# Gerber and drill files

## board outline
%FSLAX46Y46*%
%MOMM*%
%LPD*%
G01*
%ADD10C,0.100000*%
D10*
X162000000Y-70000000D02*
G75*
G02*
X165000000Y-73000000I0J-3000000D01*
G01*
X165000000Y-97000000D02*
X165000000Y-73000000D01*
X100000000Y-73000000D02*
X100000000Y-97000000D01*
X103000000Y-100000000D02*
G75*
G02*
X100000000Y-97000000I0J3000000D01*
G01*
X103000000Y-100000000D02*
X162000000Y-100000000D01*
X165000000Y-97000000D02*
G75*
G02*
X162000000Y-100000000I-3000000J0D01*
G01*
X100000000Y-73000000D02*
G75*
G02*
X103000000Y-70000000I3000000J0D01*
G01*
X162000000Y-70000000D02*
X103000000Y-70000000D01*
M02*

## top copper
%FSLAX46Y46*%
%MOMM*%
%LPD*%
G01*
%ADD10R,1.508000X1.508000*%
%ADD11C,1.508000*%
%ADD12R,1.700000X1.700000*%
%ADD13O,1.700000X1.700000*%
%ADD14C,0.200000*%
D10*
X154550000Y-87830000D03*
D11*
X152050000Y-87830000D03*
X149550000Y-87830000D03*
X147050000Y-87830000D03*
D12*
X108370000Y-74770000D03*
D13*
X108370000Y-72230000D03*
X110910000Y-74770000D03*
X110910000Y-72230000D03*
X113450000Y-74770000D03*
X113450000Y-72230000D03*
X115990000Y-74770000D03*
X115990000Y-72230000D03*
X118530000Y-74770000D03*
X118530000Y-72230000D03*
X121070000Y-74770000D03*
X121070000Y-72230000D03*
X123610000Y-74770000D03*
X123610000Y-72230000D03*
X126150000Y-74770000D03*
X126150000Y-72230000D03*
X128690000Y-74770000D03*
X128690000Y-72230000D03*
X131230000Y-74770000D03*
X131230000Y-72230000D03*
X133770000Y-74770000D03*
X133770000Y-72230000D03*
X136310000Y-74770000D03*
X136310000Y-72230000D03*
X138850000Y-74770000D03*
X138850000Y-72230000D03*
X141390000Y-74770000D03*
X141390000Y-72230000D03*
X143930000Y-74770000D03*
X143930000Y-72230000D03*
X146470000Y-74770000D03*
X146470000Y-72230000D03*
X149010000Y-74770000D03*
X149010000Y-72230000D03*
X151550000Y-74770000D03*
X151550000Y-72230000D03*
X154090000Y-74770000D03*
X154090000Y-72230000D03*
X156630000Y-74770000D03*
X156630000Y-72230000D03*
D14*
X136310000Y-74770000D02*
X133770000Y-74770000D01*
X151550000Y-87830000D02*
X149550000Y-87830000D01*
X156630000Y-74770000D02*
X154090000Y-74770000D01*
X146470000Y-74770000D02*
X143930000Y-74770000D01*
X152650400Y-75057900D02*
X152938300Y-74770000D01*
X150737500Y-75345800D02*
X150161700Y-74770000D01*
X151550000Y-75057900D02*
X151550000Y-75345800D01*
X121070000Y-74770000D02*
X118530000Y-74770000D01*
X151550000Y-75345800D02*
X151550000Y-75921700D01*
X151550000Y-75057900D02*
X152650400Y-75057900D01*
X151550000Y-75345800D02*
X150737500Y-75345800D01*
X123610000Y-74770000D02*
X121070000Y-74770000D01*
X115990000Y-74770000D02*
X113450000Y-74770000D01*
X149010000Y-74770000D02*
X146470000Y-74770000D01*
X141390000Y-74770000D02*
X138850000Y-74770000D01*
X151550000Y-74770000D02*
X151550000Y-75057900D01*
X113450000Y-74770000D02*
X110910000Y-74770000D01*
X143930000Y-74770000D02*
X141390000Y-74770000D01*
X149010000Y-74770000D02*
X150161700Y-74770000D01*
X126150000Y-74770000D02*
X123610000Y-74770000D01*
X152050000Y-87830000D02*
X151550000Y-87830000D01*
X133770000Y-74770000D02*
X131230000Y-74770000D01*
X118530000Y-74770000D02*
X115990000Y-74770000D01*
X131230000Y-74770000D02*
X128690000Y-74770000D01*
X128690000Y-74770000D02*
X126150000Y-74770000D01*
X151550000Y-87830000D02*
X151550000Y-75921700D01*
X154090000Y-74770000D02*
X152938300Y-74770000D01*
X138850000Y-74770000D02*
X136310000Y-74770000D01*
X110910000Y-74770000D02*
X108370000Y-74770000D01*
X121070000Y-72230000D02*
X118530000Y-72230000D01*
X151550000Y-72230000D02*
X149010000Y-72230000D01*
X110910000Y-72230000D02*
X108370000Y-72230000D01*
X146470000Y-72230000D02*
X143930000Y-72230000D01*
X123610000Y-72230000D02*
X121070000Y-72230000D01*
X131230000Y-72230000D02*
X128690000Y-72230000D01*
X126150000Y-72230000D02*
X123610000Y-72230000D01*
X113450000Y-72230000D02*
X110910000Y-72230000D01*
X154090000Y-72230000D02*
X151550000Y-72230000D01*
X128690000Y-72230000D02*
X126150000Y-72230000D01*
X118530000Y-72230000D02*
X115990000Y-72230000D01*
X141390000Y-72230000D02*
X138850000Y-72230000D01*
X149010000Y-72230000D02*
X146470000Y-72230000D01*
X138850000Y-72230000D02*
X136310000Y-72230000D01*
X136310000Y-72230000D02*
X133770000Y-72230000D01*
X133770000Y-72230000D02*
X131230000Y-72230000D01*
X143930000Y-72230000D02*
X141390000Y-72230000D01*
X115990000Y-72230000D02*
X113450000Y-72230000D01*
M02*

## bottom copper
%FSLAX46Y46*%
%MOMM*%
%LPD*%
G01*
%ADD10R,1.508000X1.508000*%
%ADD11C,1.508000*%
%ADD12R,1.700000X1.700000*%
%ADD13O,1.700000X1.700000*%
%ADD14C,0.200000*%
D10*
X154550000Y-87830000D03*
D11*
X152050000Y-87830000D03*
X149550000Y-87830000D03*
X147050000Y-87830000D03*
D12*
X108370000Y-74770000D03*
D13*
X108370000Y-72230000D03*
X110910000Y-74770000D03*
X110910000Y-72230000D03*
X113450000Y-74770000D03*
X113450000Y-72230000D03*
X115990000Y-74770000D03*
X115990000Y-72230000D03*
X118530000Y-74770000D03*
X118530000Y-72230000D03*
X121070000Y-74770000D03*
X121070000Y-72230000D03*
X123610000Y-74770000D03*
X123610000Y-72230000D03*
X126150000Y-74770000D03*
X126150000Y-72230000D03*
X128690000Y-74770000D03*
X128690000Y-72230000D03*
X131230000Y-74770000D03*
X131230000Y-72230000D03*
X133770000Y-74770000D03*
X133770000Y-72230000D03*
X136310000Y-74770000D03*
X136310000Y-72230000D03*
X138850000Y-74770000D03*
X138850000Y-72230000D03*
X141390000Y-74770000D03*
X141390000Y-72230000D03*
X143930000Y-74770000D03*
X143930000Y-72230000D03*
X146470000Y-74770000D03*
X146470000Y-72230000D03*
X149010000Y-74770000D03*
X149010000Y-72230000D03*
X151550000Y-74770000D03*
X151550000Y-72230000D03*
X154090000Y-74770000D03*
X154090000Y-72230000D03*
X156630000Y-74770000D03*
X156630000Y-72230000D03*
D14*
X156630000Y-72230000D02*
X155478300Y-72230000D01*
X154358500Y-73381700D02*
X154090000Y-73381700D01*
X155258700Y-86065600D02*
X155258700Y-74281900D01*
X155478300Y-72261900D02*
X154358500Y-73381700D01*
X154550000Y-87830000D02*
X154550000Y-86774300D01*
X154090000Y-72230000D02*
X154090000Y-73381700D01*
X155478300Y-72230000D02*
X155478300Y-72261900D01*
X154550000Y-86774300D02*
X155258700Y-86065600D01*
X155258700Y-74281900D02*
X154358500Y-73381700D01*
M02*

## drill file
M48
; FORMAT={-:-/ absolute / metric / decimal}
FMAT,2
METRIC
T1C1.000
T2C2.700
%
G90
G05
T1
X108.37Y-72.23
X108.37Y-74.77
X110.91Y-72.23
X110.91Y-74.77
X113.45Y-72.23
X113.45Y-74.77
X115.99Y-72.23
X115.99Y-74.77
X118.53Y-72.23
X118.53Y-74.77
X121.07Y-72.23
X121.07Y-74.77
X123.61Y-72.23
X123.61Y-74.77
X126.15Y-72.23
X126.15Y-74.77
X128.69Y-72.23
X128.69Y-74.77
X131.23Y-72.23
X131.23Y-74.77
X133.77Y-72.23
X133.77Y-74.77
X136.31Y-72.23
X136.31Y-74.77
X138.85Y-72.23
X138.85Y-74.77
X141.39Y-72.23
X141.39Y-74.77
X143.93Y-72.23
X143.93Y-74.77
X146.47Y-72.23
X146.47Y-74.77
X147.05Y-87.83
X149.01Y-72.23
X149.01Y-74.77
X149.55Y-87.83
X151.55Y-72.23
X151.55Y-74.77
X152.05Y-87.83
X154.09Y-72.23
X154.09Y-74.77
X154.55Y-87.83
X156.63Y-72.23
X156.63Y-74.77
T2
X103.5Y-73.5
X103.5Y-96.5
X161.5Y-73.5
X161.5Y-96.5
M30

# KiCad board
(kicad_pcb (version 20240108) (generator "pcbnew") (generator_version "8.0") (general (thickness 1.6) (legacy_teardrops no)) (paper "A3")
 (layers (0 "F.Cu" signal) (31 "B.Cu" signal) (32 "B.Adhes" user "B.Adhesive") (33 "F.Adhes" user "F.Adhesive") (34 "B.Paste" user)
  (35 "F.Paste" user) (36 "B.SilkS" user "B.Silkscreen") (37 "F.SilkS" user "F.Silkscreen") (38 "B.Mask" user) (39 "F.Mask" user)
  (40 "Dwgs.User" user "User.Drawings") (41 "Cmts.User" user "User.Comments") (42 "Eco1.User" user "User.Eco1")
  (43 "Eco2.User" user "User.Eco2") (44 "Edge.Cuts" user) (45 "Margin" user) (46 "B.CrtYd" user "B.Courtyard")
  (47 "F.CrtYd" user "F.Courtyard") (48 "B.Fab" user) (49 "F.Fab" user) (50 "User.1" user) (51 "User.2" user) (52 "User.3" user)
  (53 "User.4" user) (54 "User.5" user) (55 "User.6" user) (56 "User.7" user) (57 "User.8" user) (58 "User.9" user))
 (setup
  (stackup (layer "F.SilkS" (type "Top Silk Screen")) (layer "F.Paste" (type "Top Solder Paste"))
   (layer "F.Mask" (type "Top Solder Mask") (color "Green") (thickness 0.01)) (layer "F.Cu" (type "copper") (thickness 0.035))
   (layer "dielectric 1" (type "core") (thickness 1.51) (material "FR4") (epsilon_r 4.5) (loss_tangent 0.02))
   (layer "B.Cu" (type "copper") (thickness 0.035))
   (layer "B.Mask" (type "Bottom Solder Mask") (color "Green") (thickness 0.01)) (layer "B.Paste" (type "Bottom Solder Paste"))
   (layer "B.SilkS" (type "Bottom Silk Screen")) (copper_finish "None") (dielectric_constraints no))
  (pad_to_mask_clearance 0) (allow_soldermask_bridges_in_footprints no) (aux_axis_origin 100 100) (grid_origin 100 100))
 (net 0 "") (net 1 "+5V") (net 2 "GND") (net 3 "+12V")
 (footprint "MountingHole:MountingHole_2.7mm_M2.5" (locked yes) (layer "F.Cu") (at 161.5 73.5)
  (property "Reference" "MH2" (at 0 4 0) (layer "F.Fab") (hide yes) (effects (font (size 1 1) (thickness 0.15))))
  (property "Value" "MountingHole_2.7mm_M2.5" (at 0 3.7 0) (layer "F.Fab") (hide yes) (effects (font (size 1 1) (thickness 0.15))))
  (pad "" np_thru_hole circle (at 0 0) (size 2.7 2.7) (drill 2.7) (layers "*.Cu" "*.Mask")))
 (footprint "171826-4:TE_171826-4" (layer "F.Cu") (at 150.8 92.38)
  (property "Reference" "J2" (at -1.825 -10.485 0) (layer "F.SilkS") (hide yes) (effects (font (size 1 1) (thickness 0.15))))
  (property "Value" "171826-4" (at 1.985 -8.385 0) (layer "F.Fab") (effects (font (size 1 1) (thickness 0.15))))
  (pad "1" thru_hole rect (at 3.75 -4.55) (size 1.508 1.508) (drill 1) (layers "*.Cu" "*.Mask") (remove_unused_layers no) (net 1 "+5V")
   (solder_mask_margin 0.102))
  (pad "2" thru_hole circle (at 1.25 -4.55) (size 1.508 1.508) (drill 1) (layers "*.Cu" "*.Mask") (remove_unused_layers no) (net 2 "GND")
   (solder_mask_margin 0.102))
  (pad "3" thru_hole circle (at -1.25 -4.55) (size 1.508 1.508) (drill 1) (layers "*.Cu" "*.Mask") (remove_unused_layers no) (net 2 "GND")
   (solder_mask_margin 0.102))
  (pad "4" thru_hole circle (at -3.75 -4.55) (size 1.508 1.508) (drill 1) (layers "*.Cu" "*.Mask") (remove_unused_layers no) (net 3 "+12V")
   (solder_mask_margin 0.102)))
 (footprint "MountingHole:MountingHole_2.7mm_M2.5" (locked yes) (layer "F.Cu") (at 103.5 96.5)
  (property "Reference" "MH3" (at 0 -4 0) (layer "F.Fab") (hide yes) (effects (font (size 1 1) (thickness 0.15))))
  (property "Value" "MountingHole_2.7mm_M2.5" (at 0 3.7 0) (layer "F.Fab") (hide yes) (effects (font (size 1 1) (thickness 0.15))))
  (pad "" np_thru_hole circle (at 0 0) (size 2.7 2.7) (drill 2.7) (layers "*.Cu" "*.Mask")))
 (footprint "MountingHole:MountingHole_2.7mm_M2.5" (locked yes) (layer "F.Cu") (at 103.5 73.5)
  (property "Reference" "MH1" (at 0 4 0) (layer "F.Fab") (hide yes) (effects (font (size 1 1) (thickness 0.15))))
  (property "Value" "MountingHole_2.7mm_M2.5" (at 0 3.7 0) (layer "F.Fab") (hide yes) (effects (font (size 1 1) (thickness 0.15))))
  (pad "" np_thru_hole circle (at 0 0) (size 2.7 2.7) (drill 2.7) (layers "*.Cu" "*.Mask")))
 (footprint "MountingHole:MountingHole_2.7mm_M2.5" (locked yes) (layer "F.Cu") (at 161.5 96.5)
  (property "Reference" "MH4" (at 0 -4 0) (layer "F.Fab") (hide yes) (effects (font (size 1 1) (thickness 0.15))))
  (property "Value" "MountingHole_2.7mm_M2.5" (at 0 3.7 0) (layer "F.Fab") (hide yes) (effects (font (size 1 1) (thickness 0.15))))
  (pad "" np_thru_hole circle (at 0 0) (size 2.7 2.7) (drill 2.7) (layers "*.Cu" "*.Mask")))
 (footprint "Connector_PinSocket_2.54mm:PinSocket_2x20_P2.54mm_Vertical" (layer "B.Cu") (at 108.37 74.77 -90)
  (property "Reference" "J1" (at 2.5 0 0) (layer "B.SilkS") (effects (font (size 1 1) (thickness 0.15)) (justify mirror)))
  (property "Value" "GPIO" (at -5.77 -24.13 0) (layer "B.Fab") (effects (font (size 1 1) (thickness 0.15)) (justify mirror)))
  (pad "1" thru_hole rect (at 0 0 270) (size 1.7 1.7) (drill 1) (layers "*.Cu" "*.Mask") (remove_unused_layers no) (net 2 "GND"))
  (pad "2" thru_hole oval (at -2.54 0 270) (size 1.7 1.7) (drill 1) (layers "*.Cu" "*.Mask") (remove_unused_layers no) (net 1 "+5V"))
  (pad "3" thru_hole oval (at 0 -2.54 270) (size 1.7 1.7) (drill 1) (layers "*.Cu" "*.Mask") (remove_unused_layers no) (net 2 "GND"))
  (pad "4" thru_hole oval (at -2.54 -2.54 270) (size 1.7 1.7) (drill 1) (layers "*.Cu" "*.Mask") (remove_unused_layers no) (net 1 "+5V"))
  (pad "5" thru_hole oval (at 0 -5.08 270) (size 1.7 1.7) (drill 1) (layers "*.Cu" "*.Mask") (remove_unused_layers no) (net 2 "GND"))
  (pad "6" thru_hole oval (at -2.54 -5.08 270) (size 1.7 1.7) (drill 1) (layers "*.Cu" "*.Mask") (remove_unused_layers no) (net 1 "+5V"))
  (pad "7" thru_hole oval (at 0 -7.62 270) (size 1.7 1.7) (drill 1) (layers "*.Cu" "*.Mask") (remove_unused_layers no) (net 2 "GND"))
  (pad "8" thru_hole oval (at -2.54 -7.62 270) (size 1.7 1.7) (drill 1) (layers "*.Cu" "*.Mask") (remove_unused_layers no) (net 1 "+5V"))
  (pad "9" thru_hole oval (at 0 -10.16 270) (size 1.7 1.7) (drill 1) (layers "*.Cu" "*.Mask") (remove_unused_layers no) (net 2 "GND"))
  (pad "10" thru_hole oval (at -2.54 -10.16 270) (size 1.7 1.7) (drill 1) (layers "*.Cu" "*.Mask") (remove_unused_layers no) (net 1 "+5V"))
  (pad "11" thru_hole oval (at 0 -12.7 270) (size 1.7 1.7) (drill 1) (layers "*.Cu" "*.Mask") (remove_unused_layers no) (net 2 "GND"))
  (pad "12" thru_hole oval (at -2.54 -12.7 270) (size 1.7 1.7) (drill 1) (layers "*.Cu" "*.Mask") (remove_unused_layers no) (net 1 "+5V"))
  (pad "13" thru_hole oval (at 0 -15.24 270) (size 1.7 1.7) (drill 1) (layers "*.Cu" "*.Mask") (remove_unused_layers no) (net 2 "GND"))
  (pad "14" thru_hole oval (at -2.54 -15.24 270) (size 1.7 1.7) (drill 1) (layers "*.Cu" "*.Mask") (remove_unused_layers no) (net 1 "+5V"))
  (pad "15" thru_hole oval (at 0 -17.78 270) (size 1.7 1.7) (drill 1) (layers "*.Cu" "*.Mask") (remove_unused_layers no) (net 2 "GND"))
  (pad "16" thru_hole oval (at -2.54 -17.78 270) (size 1.7 1.7) (drill 1) (layers "*.Cu" "*.Mask") (remove_unused_layers no) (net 1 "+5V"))
  (pad "17" thru_hole oval (at 0 -20.32 270) (size 1.7 1.7) (drill 1) (layers "*.Cu" "*.Mask") (remove_unused_layers no) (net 2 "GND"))
  (pad "18" thru_hole oval (at -2.54 -20.32 270) (size 1.7 1.7) (drill 1) (layers "*.Cu" "*.Mask") (remove_unused_layers no) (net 1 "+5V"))
  (pad "19" thru_hole oval (at 0 -22.86 270) (size 1.7 1.7) (drill 1) (layers "*.Cu" "*.Mask") (remove_unused_layers no) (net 2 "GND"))
  (pad "20" thru_hole oval (at -2.54 -22.86 270) (size 1.7 1.7) (drill 1) (layers "*.Cu" "*.Mask") (remove_unused_layers no) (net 1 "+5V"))
  (pad "21" thru_hole oval (at 0 -25.4 270) (size 1.7 1.7) (drill 1) (layers "*.Cu" "*.Mask") (remove_unused_layers no) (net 2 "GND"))
  (pad "22" thru_hole oval (at -2.54 -25.4 270) (size 1.7 1.7) (drill 1) (layers "*.Cu" "*.Mask") (remove_unused_layers no) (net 1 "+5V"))
  (pad "23" thru_hole oval (at 0 -27.94 270) (size 1.7 1.7) (drill 1) (layers "*.Cu" "*.Mask") (remove_unused_layers no) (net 2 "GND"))
  (pad "24" thru_hole oval (at -2.54 -27.94 270) (size 1.7 1.7) (drill 1) (layers "*.Cu" "*.Mask") (remove_unused_layers no) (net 1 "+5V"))
  (pad "25" thru_hole oval (at 0 -30.48 270) (size 1.7 1.7) (drill 1) (layers "*.Cu" "*.Mask") (remove_unused_layers no) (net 2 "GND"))
  (pad "26" thru_hole oval (at -2.54 -30.48 270) (size 1.7 1.7) (drill 1) (layers "*.Cu" "*.Mask") (remove_unused_layers no) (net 1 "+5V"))
  (pad "27" thru_hole oval (at 0 -33.02 270) (size 1.7 1.7) (drill 1) (layers "*.Cu" "*.Mask") (remove_unused_layers no) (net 2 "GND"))
  (pad "28" thru_hole oval (at -2.54 -33.02 270) (size 1.7 1.7) (drill 1) (layers "*.Cu" "*.Mask") (remove_unused_layers no) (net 1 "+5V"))
  (pad "29" thru_hole oval (at 0 -35.56 270) (size 1.7 1.7) (drill 1) (layers "*.Cu" "*.Mask") (remove_unused_layers no) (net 2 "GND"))
  (pad "30" thru_hole oval (at -2.54 -35.56 270) (size 1.7 1.7) (drill 1) (layers "*.Cu" "*.Mask") (remove_unused_layers no) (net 1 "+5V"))
  (pad "31" thru_hole oval (at 0 -38.1 270) (size 1.7 1.7) (drill 1) (layers "*.Cu" "*.Mask") (remove_unused_layers no) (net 2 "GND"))
  (pad "32" thru_hole oval (at -2.54 -38.1 270) (size 1.7 1.7) (drill 1) (layers "*.Cu" "*.Mask") (remove_unused_layers no) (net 1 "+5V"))
  (pad "33" thru_hole oval (at 0 -40.64 270) (size 1.7 1.7) (drill 1) (layers "*.Cu" "*.Mask") (remove_unused_layers no) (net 2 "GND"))
  (pad "34" thru_hole oval (at -2.54 -40.64 270) (size 1.7 1.7) (drill 1) (layers "*.Cu" "*.Mask") (remove_unused_layers no) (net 1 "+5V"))
  (pad "35" thru_hole oval (at 0 -43.18 270) (size 1.7 1.7) (drill 1) (layers "*.Cu" "*.Mask") (remove_unused_layers no) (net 2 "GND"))
  (pad "36" thru_hole oval (at -2.54 -43.18 270) (size 1.7 1.7) (drill 1) (layers "*.Cu" "*.Mask") (remove_unused_layers no) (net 1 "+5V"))
  (pad "37" thru_hole oval (at 0 -45.72 270) (size 1.7 1.7) (drill 1) (layers "*.Cu" "*.Mask") (remove_unused_layers no) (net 2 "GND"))
  (pad "38" thru_hole oval (at -2.54 -45.72 270) (size 1.7 1.7) (drill 1) (layers "*.Cu" "*.Mask") (remove_unused_layers no) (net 1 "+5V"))
  (pad "39" thru_hole oval (at 0 -48.26 270) (size 1.7 1.7) (drill 1) (layers "*.Cu" "*.Mask") (remove_unused_layers no) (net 2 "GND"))
  (pad "40" thru_hole oval (at -2.54 -48.26 270) (size 1.7 1.7) (drill 1) (layers "*.Cu" "*.Mask") (remove_unused_layers no) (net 1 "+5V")))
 (gr_arc (start 162 70) (mid 164.12132 70.87868) (end 165 73) (stroke (width 0.1) (type solid)) (layer "Edge.Cuts"))
 (gr_line (start 165 97) (end 165 73) (stroke (width 0.1) (type solid)) (layer "Edge.Cuts"))
 (gr_line (start 100 73) (end 100 97) (stroke (width 0.1) (type solid)) (layer "Edge.Cuts"))
 (gr_arc (start 103 100) (mid 100.87868 99.12132) (end 100 97) (stroke (width 0.1) (type solid)) (layer "Edge.Cuts"))
 (gr_line (start 103 100) (end 162 100) (stroke (width 0.1) (type solid)) (layer "Edge.Cuts"))
 (gr_arc (start 165 97) (mid 164.12132 99.12132) (end 162 100) (stroke (width 0.1) (type solid)) (layer "Edge.Cuts"))
 (gr_arc (start 100 73) (mid 100.87868 70.87868) (end 103 70) (stroke (width 0.1) (type solid)) (layer "Edge.Cuts"))
 (gr_line (start 162 70) (end 103 70) (stroke (width 0.1) (type solid)) (layer "Edge.Cuts"))
 (segment (start 136.31 74.77) (end 133.77 74.77) (width 0.2) (layer "F.Cu") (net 2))
 (segment (start 151.55 87.83) (end 149.55 87.83) (width 0.2) (layer "F.Cu") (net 2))
 (segment (start 156.63 74.77) (end 154.09 74.77) (width 0.2) (layer "F.Cu") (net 2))
 (segment (start 146.47 74.77) (end 143.93 74.77) (width 0.2) (layer "F.Cu") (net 2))
 (segment (start 152.6504 75.0579) (end 152.9383 74.77) (width 0.2) (layer "F.Cu") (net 2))
 (segment (start 150.7375 75.3458) (end 150.1617 74.77) (width 0.2) (layer "F.Cu") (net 2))
 (segment (start 151.55 75.0579) (end 151.55 75.3458) (width 0.2) (layer "F.Cu") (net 2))
 (segment (start 121.07 74.77) (end 118.53 74.77) (width 0.2) (layer "F.Cu") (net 2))
 (segment (start 151.55 75.3458) (end 151.55 75.9217) (width 0.2) (layer "F.Cu") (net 2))
 (segment (start 151.55 75.0579) (end 152.6504 75.0579) (width 0.2) (layer "F.Cu") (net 2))
 (segment (start 151.55 75.3458) (end 150.7375 75.3458) (width 0.2) (layer "F.Cu") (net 2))
 (segment (start 123.61 74.77) (end 121.07 74.77) (width 0.2) (layer "F.Cu") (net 2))
 (segment (start 115.99 74.77) (end 113.45 74.77) (width 0.2) (layer "F.Cu") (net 2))
 (segment (start 149.01 74.77) (end 146.47 74.77) (width 0.2) (layer "F.Cu") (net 2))
 (segment (start 141.39 74.77) (end 138.85 74.77) (width 0.2) (layer "F.Cu") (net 2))
 (segment (start 151.55 74.77) (end 151.55 75.0579) (width 0.2) (layer "F.Cu") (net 2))
 (segment (start 113.45 74.77) (end 110.91 74.77) (width 0.2) (layer "F.Cu") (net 2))
 (segment (start 143.93 74.77) (end 141.39 74.77) (width 0.2) (layer "F.Cu") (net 2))
 (segment (start 149.01 74.77) (end 150.1617 74.77) (width 0.2) (layer "F.Cu") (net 2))
 (segment (start 126.15 74.77) (end 123.61 74.77) (width 0.2) (layer "F.Cu") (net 2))
 (segment (start 152.05 87.83) (end 151.55 87.83) (width 0.2) (layer "F.Cu") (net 2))
 (segment (start 133.77 74.77) (end 131.23 74.77) (width 0.2) (layer "F.Cu") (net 2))
 (segment (start 118.53 74.77) (end 115.99 74.77) (width 0.2) (layer "F.Cu") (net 2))
 (segment (start 131.23 74.77) (end 128.69 74.77) (width 0.2) (layer "F.Cu") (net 2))
 (segment (start 128.69 74.77) (end 126.15 74.77) (width 0.2) (layer "F.Cu") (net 2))
 (segment (start 151.55 87.83) (end 151.55 75.9217) (width 0.2) (layer "F.Cu") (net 2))
 (segment (start 154.09 74.77) (end 152.9383 74.77) (width 0.2) (layer "F.Cu") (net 2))
 (segment (start 138.85 74.77) (end 136.31 74.77) (width 0.2) (layer "F.Cu") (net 2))
 (segment (start 110.91 74.77) (end 108.37 74.77) (width 0.2) (layer "F.Cu") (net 2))
 (segment (start 121.07 72.23) (end 118.53 72.23) (width 0.2) (layer "F.Cu") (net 1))
 (segment (start 151.55 72.23) (end 149.01 72.23) (width 0.2) (layer "F.Cu") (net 1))
 (segment (start 110.91 72.23) (end 108.37 72.23) (width 0.2) (layer "F.Cu") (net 1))
 (segment (start 146.47 72.23) (end 143.93 72.23) (width 0.2) (layer "F.Cu") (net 1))
 (segment (start 123.61 72.23) (end 121.07 72.23) (width 0.2) (layer "F.Cu") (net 1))
 (segment (start 131.23 72.23) (end 128.69 72.23) (width 0.2) (layer "F.Cu") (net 1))
 (segment (start 126.15 72.23) (end 123.61 72.23) (width 0.2) (layer "F.Cu") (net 1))
 (segment (start 113.45 72.23) (end 110.91 72.23) (width 0.2) (layer "F.Cu") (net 1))
 (segment (start 154.09 72.23) (end 151.55 72.23) (width 0.2) (layer "F.Cu") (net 1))
 (segment (start 128.69 72.23) (end 126.15 72.23) (width 0.2) (layer "F.Cu") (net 1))
 (segment (start 118.53 72.23) (end 115.99 72.23) (width 0.2) (layer "F.Cu") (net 1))
 (segment (start 141.39 72.23) (end 138.85 72.23) (width 0.2) (layer "F.Cu") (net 1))
 (segment (start 149.01 72.23) (end 146.47 72.23) (width 0.2) (layer "F.Cu") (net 1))
 (segment (start 138.85 72.23) (end 136.31 72.23) (width 0.2) (layer "F.Cu") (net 1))
 (segment (start 136.31 72.23) (end 133.77 72.23) (width 0.2) (layer "F.Cu") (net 1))
 (segment (start 133.77 72.23) (end 131.23 72.23) (width 0.2) (layer "F.Cu") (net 1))
 (segment (start 143.93 72.23) (end 141.39 72.23) (width 0.2) (layer "F.Cu") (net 1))
 (segment (start 115.99 72.23) (end 113.45 72.23) (width 0.2) (layer "F.Cu") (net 1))
 (segment (start 156.63 72.23) (end 155.4783 72.23) (width 0.2) (layer "B.Cu") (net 1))
 (segment (start 154.3585 73.3817) (end 154.09 73.3817) (width 0.2) (layer "B.Cu") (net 1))
 (segment (start 155.2587 86.0656) (end 155.2587 74.2819) (width 0.2) (layer "B.Cu") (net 1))
 (segment (start 155.4783 72.2619) (end 154.3585 73.3817) (width 0.2) (layer "B.Cu") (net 1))
 (segment (start 154.55 87.83) (end 154.55 86.7743) (width 0.2) (layer "B.Cu") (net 1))
 (segment (start 154.09 72.23) (end 154.09 73.3817) (width 0.2) (layer "B.Cu") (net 1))
 (segment (start 155.4783 72.23) (end 155.4783 72.2619) (width 0.2) (layer "B.Cu") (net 1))
 (segment (start 154.55 86.7743) (end 155.2587 86.0656) (width 0.2) (layer "B.Cu") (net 1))
 (segment (start 155.2587 74.2819) (end 154.3585 73.3817) (width 0.2) (layer "B.Cu") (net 1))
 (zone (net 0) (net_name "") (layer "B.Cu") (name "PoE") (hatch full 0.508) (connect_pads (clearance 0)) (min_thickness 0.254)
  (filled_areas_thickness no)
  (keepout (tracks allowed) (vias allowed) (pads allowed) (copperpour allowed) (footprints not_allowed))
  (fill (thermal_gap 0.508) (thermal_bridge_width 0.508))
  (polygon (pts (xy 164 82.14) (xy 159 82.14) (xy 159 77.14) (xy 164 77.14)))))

